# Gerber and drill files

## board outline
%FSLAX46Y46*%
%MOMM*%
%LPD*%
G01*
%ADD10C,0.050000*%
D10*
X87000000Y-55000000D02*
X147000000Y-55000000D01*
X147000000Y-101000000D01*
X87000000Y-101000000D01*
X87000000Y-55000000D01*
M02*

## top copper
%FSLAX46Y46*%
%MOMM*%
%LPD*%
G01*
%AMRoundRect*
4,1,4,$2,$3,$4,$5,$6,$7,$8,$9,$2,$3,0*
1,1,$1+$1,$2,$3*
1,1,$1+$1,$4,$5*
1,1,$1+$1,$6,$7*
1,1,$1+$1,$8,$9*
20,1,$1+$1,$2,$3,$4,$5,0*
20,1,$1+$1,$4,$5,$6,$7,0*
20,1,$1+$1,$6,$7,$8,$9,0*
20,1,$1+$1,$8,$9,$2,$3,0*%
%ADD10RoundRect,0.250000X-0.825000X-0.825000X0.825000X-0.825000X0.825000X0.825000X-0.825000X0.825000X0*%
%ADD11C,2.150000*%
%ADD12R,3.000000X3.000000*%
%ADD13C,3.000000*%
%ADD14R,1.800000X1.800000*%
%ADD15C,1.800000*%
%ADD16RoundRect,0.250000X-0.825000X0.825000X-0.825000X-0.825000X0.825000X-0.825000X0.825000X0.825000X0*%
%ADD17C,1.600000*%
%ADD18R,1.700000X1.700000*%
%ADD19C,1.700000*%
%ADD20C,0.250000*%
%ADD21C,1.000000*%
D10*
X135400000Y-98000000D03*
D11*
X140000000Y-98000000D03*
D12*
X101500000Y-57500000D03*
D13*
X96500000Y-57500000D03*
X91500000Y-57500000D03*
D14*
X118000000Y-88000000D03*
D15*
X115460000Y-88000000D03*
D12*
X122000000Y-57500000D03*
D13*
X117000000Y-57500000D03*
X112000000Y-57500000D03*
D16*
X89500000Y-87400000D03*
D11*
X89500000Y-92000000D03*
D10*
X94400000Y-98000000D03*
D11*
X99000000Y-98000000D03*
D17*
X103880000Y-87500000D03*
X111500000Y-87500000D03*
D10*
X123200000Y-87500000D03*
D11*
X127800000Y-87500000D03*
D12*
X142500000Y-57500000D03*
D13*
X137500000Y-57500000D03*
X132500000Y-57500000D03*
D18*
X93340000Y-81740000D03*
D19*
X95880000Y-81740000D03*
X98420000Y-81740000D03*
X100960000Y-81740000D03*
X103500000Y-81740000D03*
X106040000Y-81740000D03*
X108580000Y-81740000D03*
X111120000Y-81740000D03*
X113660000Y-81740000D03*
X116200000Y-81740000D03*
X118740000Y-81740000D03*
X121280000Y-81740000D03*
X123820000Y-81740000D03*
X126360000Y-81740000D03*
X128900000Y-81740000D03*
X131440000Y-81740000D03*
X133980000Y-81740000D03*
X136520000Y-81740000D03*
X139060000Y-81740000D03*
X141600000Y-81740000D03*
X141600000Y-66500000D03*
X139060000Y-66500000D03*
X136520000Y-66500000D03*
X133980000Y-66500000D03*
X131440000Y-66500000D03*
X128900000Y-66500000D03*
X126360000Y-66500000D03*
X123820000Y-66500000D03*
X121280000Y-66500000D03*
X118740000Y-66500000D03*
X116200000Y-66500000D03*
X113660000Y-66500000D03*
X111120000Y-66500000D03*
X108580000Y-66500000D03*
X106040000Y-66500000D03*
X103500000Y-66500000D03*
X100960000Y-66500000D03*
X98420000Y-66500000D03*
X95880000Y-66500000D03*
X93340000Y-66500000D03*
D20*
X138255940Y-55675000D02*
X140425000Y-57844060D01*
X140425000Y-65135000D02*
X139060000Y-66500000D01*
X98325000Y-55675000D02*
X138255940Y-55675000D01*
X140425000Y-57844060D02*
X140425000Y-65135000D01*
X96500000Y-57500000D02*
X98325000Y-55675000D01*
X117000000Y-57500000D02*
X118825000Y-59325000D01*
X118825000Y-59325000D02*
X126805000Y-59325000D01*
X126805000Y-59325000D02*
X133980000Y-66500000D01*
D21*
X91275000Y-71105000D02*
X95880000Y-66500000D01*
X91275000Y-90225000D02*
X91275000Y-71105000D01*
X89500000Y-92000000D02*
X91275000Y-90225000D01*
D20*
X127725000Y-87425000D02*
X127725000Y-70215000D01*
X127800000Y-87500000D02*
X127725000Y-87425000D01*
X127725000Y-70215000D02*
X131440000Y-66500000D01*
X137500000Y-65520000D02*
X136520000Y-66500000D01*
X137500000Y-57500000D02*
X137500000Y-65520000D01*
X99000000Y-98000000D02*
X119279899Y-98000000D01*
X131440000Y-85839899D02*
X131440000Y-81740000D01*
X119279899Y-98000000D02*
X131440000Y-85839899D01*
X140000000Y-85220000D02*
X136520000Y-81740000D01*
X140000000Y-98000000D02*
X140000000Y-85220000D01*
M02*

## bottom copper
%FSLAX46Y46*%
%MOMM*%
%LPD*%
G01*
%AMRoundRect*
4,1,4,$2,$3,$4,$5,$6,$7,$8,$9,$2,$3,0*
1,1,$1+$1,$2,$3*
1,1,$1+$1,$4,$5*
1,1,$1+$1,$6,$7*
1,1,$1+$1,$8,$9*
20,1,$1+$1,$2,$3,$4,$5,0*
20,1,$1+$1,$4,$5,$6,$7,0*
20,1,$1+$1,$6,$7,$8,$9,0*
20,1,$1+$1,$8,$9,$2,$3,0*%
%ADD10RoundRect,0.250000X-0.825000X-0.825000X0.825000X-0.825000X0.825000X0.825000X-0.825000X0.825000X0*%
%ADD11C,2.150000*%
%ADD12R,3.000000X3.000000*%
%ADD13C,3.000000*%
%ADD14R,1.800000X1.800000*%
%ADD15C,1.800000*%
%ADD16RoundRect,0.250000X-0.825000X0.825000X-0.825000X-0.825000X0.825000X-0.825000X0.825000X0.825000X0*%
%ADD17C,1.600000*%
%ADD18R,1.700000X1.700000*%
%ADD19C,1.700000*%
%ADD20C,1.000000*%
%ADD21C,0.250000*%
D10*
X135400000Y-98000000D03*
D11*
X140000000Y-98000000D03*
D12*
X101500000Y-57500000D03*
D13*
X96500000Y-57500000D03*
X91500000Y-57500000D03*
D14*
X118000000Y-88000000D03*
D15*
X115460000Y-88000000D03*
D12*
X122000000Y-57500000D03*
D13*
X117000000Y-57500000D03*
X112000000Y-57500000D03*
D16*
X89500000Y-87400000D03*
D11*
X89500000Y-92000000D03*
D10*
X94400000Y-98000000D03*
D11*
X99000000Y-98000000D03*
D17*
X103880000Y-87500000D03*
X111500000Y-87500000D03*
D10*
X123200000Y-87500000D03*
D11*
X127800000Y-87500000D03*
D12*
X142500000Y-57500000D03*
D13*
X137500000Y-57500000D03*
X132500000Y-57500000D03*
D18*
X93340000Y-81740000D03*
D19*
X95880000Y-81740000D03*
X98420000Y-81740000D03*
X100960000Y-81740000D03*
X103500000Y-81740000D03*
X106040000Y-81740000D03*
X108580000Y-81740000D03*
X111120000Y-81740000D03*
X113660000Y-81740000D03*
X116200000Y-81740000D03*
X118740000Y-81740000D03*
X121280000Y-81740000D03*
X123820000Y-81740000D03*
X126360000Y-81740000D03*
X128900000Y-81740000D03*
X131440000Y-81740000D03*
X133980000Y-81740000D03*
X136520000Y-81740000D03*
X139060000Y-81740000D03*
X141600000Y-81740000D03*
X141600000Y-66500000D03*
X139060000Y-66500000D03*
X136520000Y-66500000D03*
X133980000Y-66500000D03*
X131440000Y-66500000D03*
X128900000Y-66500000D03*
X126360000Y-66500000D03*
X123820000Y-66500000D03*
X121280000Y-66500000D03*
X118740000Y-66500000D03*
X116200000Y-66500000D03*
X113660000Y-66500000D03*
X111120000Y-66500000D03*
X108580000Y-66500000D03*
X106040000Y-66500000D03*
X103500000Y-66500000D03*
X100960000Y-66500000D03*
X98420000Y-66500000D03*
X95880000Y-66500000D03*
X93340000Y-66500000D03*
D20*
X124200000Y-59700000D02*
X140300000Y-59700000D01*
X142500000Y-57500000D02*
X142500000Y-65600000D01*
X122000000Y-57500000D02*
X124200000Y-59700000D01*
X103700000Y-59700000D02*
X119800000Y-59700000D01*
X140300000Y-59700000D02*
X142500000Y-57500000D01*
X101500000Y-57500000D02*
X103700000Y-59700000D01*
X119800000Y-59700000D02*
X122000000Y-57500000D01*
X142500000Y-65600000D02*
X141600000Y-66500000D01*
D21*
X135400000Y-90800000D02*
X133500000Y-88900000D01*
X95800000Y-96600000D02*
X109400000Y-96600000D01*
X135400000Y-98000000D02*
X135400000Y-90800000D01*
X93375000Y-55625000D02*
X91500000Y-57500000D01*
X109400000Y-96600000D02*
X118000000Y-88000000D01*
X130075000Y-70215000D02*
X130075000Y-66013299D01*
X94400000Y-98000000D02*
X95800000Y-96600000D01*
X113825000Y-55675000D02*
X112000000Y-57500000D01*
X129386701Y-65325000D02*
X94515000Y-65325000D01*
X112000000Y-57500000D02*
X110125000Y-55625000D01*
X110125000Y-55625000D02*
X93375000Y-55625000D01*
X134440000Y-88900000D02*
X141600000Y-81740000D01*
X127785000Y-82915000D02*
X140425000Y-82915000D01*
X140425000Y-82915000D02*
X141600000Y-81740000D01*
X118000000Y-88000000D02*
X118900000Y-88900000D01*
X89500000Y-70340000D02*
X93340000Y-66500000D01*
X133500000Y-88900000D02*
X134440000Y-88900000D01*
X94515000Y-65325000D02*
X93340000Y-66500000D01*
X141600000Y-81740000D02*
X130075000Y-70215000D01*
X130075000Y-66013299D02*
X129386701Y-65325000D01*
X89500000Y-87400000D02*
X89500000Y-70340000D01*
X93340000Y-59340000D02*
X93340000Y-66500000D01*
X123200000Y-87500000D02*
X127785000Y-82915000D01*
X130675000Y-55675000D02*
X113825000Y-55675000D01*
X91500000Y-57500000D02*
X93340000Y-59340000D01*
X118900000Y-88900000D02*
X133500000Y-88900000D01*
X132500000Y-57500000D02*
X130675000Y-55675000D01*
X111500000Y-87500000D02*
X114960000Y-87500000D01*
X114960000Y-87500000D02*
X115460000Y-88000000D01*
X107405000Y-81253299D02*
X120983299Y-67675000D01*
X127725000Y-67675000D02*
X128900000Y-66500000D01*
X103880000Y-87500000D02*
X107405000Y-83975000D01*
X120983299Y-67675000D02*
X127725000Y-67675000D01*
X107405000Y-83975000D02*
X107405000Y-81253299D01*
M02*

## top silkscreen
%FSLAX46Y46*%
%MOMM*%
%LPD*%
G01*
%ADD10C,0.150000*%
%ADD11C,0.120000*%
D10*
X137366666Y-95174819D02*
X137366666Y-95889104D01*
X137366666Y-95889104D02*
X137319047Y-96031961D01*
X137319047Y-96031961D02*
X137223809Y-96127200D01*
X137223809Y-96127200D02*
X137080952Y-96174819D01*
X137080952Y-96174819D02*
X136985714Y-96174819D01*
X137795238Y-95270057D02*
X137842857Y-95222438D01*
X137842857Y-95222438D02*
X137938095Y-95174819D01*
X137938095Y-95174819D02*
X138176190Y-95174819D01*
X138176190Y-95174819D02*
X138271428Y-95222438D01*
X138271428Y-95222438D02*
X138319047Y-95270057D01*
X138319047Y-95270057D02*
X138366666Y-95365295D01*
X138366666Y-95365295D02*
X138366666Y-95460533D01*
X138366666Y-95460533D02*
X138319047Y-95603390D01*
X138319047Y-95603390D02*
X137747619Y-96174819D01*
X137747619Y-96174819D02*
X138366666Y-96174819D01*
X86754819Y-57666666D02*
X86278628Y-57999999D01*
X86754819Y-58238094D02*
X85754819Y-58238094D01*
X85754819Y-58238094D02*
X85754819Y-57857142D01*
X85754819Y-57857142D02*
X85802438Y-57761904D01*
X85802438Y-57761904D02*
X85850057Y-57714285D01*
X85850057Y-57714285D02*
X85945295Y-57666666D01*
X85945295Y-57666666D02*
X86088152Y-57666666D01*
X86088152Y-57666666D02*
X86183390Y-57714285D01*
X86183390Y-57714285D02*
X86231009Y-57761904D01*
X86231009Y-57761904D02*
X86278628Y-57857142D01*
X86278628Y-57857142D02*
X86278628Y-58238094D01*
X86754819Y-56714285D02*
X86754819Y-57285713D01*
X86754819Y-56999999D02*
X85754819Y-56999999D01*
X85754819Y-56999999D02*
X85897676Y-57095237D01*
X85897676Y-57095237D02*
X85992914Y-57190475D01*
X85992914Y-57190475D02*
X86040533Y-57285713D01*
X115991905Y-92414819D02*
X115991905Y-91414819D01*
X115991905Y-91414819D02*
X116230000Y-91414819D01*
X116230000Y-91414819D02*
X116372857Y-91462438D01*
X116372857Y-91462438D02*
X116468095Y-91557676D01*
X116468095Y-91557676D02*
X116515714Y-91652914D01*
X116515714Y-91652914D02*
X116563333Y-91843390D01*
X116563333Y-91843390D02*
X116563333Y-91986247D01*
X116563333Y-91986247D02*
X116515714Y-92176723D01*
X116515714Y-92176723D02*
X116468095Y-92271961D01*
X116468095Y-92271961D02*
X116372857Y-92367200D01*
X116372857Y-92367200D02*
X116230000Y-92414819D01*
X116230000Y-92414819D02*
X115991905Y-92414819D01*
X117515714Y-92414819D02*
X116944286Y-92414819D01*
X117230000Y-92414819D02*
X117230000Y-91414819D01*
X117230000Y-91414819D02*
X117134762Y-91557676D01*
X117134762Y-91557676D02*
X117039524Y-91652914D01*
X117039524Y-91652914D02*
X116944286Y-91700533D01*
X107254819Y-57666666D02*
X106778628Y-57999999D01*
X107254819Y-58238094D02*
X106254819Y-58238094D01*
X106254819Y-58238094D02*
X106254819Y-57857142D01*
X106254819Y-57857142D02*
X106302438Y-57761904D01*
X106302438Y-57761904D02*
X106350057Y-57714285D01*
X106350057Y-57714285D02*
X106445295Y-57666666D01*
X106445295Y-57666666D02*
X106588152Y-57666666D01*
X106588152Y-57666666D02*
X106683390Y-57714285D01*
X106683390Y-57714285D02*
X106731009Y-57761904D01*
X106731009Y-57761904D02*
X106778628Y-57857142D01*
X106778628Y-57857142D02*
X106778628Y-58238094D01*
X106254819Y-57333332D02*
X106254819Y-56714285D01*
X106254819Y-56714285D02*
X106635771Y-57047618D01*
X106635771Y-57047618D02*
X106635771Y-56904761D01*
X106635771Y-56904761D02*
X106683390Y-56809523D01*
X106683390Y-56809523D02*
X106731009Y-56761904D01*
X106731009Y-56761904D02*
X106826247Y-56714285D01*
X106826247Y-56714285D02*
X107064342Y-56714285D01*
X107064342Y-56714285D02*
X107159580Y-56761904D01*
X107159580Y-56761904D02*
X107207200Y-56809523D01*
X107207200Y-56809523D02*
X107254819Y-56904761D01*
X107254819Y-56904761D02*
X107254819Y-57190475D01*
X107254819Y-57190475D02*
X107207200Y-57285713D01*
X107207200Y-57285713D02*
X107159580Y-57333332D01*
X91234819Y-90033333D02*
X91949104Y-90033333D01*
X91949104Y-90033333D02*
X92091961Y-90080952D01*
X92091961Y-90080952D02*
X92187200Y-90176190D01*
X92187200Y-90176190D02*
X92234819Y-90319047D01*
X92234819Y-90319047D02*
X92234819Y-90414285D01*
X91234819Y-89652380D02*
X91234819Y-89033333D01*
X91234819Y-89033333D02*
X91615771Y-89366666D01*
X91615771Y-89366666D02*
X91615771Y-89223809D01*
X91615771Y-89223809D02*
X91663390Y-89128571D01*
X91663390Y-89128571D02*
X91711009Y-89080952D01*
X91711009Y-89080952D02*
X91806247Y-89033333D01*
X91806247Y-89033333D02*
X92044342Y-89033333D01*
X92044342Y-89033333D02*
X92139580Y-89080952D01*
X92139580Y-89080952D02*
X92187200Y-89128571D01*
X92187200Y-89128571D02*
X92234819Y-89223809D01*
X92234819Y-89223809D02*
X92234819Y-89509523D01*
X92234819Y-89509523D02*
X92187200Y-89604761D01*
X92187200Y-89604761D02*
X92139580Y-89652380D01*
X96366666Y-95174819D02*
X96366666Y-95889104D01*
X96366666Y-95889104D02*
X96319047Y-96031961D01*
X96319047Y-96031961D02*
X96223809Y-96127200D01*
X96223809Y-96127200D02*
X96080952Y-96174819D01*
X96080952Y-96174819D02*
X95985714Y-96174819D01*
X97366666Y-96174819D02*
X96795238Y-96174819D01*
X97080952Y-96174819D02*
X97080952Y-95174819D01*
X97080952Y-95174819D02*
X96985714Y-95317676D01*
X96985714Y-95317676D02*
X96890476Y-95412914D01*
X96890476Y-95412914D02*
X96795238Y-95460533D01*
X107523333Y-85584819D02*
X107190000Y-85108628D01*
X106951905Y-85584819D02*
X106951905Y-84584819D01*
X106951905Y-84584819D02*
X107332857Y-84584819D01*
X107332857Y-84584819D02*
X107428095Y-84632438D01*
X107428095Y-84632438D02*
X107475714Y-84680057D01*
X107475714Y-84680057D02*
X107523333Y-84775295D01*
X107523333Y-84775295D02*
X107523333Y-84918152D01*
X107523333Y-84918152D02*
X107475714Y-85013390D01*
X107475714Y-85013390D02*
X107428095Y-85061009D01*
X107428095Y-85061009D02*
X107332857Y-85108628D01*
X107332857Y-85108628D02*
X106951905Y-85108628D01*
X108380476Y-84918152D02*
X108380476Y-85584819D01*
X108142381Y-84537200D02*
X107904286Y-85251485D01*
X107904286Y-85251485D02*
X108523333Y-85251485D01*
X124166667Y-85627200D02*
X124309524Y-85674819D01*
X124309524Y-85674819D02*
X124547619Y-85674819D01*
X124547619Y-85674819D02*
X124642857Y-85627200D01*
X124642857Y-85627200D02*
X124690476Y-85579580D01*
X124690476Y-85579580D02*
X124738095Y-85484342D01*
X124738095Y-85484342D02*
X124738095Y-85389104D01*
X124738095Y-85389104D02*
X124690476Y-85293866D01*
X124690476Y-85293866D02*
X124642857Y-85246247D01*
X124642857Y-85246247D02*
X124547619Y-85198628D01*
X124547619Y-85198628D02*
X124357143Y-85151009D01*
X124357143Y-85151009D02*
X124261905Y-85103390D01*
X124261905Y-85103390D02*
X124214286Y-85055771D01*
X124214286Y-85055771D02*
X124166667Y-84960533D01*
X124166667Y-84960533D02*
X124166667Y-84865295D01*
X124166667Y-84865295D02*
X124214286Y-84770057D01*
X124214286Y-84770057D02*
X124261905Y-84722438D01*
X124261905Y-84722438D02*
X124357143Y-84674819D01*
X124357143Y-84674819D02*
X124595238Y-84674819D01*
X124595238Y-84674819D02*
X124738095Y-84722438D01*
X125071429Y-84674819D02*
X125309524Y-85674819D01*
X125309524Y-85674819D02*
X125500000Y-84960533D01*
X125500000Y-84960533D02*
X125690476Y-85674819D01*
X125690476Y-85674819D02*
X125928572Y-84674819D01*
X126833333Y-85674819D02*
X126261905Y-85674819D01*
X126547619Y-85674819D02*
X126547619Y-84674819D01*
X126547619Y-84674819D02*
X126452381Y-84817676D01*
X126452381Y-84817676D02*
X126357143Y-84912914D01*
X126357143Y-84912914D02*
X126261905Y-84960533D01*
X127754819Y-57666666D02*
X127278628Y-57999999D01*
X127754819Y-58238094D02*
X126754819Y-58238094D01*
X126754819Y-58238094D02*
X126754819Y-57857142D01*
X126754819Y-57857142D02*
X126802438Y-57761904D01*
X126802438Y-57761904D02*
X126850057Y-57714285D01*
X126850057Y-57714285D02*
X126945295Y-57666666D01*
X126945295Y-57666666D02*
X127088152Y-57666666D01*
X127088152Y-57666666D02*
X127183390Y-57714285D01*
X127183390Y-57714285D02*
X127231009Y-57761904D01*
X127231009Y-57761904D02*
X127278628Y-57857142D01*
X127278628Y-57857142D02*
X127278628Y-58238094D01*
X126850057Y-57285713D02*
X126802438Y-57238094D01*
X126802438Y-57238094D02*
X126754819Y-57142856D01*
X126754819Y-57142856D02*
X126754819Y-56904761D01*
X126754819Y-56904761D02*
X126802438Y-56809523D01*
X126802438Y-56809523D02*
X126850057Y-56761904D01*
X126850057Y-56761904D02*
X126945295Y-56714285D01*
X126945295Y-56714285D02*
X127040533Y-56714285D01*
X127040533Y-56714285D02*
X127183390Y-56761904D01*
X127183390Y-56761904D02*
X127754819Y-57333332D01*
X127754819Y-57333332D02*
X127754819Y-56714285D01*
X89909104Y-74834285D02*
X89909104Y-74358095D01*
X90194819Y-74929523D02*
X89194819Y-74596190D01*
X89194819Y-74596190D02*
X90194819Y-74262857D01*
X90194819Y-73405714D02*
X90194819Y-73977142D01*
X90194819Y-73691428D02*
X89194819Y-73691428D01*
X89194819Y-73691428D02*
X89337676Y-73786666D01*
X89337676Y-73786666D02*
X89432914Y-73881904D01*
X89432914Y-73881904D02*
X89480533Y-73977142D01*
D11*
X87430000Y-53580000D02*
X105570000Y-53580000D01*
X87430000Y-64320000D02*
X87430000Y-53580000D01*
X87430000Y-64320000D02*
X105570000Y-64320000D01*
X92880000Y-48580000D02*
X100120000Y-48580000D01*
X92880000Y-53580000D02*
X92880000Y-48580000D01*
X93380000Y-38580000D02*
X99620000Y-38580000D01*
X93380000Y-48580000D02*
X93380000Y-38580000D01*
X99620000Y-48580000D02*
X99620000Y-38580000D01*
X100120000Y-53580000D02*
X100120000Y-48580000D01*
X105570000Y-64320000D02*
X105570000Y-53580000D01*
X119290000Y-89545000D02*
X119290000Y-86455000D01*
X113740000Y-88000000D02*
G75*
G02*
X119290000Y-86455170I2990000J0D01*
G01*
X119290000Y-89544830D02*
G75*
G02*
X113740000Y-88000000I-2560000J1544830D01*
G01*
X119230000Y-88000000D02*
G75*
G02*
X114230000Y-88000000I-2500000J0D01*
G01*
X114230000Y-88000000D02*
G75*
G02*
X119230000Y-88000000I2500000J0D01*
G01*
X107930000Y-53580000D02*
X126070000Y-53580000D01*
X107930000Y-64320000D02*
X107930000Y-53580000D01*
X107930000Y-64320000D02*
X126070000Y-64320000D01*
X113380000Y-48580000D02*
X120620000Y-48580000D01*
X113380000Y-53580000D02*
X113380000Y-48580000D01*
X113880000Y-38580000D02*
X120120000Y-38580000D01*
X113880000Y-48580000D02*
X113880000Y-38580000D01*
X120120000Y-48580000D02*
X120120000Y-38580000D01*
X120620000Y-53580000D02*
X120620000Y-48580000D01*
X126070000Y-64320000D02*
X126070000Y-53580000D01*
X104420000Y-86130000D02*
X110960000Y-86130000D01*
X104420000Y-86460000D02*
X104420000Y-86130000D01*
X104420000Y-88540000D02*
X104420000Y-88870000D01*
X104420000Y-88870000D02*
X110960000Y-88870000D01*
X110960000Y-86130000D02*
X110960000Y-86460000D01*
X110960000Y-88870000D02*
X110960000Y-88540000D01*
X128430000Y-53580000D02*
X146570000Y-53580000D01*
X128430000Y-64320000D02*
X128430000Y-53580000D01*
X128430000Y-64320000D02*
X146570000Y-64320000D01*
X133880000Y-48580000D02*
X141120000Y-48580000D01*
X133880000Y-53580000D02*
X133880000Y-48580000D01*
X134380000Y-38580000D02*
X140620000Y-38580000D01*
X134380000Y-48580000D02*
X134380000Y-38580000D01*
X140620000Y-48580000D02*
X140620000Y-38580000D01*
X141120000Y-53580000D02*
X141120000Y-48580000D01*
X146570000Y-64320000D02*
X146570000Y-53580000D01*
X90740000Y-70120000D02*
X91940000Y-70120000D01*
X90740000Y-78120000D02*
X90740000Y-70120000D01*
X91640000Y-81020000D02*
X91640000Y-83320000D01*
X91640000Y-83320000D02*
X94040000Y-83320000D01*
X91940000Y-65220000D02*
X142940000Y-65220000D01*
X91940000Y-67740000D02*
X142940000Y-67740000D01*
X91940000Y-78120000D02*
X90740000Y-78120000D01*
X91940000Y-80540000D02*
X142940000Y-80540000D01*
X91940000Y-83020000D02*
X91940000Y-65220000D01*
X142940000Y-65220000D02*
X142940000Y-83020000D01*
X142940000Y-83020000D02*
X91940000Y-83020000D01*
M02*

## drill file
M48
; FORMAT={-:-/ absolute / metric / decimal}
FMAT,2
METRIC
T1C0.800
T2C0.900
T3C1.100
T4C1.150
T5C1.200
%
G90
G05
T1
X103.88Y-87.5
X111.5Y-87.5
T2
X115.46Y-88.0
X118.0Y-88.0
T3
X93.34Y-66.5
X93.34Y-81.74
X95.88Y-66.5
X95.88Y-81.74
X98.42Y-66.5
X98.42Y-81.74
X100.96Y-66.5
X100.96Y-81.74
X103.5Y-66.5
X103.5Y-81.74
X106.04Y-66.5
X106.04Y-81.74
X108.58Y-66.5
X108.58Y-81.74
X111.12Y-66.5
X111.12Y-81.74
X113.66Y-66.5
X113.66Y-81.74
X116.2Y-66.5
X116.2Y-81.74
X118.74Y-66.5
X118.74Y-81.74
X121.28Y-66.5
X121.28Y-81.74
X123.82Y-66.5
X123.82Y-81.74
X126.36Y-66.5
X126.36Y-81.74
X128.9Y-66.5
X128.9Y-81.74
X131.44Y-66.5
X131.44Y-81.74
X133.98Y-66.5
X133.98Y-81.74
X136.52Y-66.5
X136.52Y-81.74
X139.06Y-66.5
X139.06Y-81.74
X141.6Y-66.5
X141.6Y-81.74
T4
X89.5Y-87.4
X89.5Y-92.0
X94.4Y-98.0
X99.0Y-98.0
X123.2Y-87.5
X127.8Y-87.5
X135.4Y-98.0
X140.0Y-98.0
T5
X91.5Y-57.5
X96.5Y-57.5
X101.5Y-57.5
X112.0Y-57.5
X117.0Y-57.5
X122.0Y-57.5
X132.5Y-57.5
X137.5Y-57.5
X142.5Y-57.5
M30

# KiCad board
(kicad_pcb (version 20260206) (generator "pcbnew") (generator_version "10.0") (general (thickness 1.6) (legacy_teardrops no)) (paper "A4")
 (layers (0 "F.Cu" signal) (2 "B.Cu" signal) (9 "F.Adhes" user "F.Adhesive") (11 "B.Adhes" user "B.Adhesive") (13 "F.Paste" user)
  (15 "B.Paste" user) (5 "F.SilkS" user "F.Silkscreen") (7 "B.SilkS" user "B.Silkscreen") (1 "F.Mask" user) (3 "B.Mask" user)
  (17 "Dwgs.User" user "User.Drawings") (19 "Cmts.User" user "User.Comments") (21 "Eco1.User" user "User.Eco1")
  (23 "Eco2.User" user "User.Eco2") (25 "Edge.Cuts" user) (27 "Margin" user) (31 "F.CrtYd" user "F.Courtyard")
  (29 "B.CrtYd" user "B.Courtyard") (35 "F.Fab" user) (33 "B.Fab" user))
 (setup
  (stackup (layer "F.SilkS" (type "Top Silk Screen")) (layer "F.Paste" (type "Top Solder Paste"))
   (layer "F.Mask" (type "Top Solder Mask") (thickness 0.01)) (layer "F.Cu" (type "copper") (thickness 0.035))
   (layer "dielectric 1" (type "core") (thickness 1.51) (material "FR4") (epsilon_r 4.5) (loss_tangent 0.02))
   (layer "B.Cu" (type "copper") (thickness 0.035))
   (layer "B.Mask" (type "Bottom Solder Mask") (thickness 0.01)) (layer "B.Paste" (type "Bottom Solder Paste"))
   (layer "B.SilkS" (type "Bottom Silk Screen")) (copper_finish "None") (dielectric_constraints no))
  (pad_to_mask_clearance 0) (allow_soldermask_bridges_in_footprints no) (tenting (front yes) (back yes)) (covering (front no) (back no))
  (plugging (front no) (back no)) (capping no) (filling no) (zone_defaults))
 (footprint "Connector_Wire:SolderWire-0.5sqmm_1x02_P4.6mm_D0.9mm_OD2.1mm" (layer "F.Cu") (at 135.4 98)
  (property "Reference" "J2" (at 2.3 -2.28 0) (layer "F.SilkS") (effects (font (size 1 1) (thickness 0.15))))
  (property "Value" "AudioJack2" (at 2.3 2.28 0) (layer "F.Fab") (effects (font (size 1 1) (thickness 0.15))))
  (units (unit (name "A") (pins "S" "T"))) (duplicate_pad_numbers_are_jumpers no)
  (pad "S" thru_hole roundrect (at 0 0) (size 2.15 2.15) (drill 1.15) (layers "*.Cu" "*.Mask") (remove_unused_layers no)
   (roundrect_rratio 0.116279) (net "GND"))
  (pad "T" thru_hole circle (at 4.6 0) (size 2.15 2.15) (drill 1.15) (layers "*.Cu" "*.Mask") (remove_unused_layers no)
   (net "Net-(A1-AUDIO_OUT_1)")))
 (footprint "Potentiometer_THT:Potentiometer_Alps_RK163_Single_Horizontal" (layer "F.Cu") (at 101.5 57.5 -90)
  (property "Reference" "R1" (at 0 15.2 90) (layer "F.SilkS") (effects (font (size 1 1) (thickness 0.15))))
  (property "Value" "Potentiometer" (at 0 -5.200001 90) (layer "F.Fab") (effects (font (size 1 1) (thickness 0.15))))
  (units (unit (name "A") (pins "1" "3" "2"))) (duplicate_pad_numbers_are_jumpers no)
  (fp_line (start -3.92 14.07) (end -3.92 -4.07) (stroke (width 0.12) (type solid)) (layer "F.SilkS"))
  (fp_line (start 6.82 14.07) (end -3.92 14.07) (stroke (width 0.12) (type solid)) (layer "F.SilkS"))
  (fp_line (start 6.82 14.07) (end 6.82 -4.07) (stroke (width 0.12) (type solid)) (layer "F.SilkS"))
  (fp_line (start -8.92 8.62) (end -8.92 1.38) (stroke (width 0.12) (type solid)) (layer "F.SilkS"))
  (fp_line (start -3.92 8.62) (end -8.92 8.62) (stroke (width 0.12) (type solid)) (layer "F.SilkS"))
  (fp_line (start -18.92 8.12) (end -18.92 1.88) (stroke (width 0.12) (type solid)) (layer "F.SilkS"))
  (fp_line (start -8.92 8.12) (end -18.92 8.12) (stroke (width 0.12) (type solid)) (layer "F.SilkS"))
  (fp_line (start -8.92 1.88) (end -18.92 1.88) (stroke (width 0.12) (type solid)) (layer "F.SilkS"))
  (fp_line (start -3.92 1.38) (end -8.92 1.38) (stroke (width 0.12) (type solid)) (layer "F.SilkS"))
  (fp_line (start 6.82 -4.07) (end -3.92 -4.07) (stroke (width 0.12) (type solid)) (layer "F.SilkS"))
  (pad "1" thru_hole rect (at 0 0 90) (size 3 3) (drill 1.2) (layers "*.Cu" "*.Mask") (remove_unused_layers no) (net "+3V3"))
  (pad "2" thru_hole circle (at 0 5 90) (size 3 3) (drill 1.2) (layers "*.Cu" "*.Mask") (remove_unused_layers no) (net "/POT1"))
  (pad "3" thru_hole circle (at 0 10 90) (size 3 3) (drill 1.2) (layers "*.Cu" "*.Mask") (remove_unused_layers no) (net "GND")))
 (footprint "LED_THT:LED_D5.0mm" (layer "F.Cu") (at 118 88 180)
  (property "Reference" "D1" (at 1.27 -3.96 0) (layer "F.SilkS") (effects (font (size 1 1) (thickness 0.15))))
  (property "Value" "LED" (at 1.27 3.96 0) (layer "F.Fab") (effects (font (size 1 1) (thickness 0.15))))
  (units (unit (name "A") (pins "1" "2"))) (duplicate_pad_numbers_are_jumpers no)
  (fp_line (start -1.29 -1.545) (end -1.29 1.545) (stroke (width 0.12) (type solid)) (layer "F.SilkS"))
  (fp_arc (start 4.26 0) (mid 2.071779 2.880495) (end -1.29 1.54483) (stroke (width 0.12) (type solid)) (layer "F.SilkS"))
  (fp_arc (start -1.29 -1.54483) (mid 2.071779 -2.880495) (end 4.26 0) (stroke (width 0.12) (type solid)) (layer "F.SilkS"))
  (fp_circle (center 1.27 0) (end 3.77 0) (stroke (width 0.12) (type solid)) (fill no) (layer "F.SilkS"))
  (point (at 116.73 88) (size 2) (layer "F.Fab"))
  (pad "1" thru_hole rect (at 0 0 180) (size 1.8 1.8) (drill 0.9) (layers "*.Cu" "*.Mask") (remove_unused_layers no) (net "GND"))
  (pad "2" thru_hole circle (at 2.54 0 180) (size 1.8 1.8) (drill 0.9) (layers "*.Cu" "*.Mask") (remove_unused_layers no) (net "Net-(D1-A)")))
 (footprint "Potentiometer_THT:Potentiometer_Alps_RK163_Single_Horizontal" (layer "F.Cu") (at 122 57.5 -90)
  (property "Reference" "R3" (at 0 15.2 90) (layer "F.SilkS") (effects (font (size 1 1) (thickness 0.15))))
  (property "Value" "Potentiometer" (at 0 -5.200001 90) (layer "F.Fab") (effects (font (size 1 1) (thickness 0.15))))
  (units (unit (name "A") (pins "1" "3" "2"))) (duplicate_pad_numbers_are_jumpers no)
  (fp_line (start -3.92 14.07) (end -3.92 -4.07) (stroke (width 0.12) (type solid)) (layer "F.SilkS"))
  (fp_line (start 6.82 14.07) (end -3.92 14.07) (stroke (width 0.12) (type solid)) (layer "F.SilkS"))
  (fp_line (start 6.82 14.07) (end 6.82 -4.07) (stroke (width 0.12) (type solid)) (layer "F.SilkS"))
  (fp_line (start -8.92 8.62) (end -8.92 1.38) (stroke (width 0.12) (type solid)) (layer "F.SilkS"))
  (fp_line (start -3.92 8.62) (end -8.92 8.62) (stroke (width 0.12) (type solid)) (layer "F.SilkS"))
  (fp_line (start -18.92 8.12) (end -18.92 1.88) (stroke (width 0.12) (type solid)) (layer "F.SilkS"))
  (fp_line (start -8.92 8.12) (end -18.92 8.12) (stroke (width 0.12) (type solid)) (layer "F.SilkS"))
  (fp_line (start -8.92 1.88) (end -18.92 1.88) (stroke (width 0.12) (type solid)) (layer "F.SilkS"))
  (fp_line (start -3.92 1.38) (end -8.92 1.38) (stroke (width 0.12) (type solid)) (layer "F.SilkS"))
  (fp_line (start 6.82 -4.07) (end -3.92 -4.07) (stroke (width 0.12) (type solid)) (layer "F.SilkS"))
  (pad "1" thru_hole rect (at 0 0 90) (size 3 3) (drill 1.2) (layers "*.Cu" "*.Mask") (remove_unused_layers no) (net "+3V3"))
  (pad "2" thru_hole circle (at 0 5 90) (size 3 3) (drill 1.2) (layers "*.Cu" "*.Mask") (remove_unused_layers no) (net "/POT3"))
  (pad "3" thru_hole circle (at 0 10 90) (size 3 3) (drill 1.2) (layers "*.Cu" "*.Mask") (remove_unused_layers no) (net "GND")))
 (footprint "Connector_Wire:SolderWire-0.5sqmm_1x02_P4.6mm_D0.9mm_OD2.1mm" (layer "F.Cu") (at 89.5 87.4 -90)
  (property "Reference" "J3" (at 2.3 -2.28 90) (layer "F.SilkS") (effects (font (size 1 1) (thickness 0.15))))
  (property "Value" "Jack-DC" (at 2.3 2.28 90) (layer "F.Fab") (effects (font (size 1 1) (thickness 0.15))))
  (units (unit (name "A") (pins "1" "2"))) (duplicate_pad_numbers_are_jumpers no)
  (pad "1" thru_hole roundrect (at 0 0 270) (size 2.15 2.15) (drill 1.15) (layers "*.Cu" "*.Mask") (remove_unused_layers no)
   (roundrect_rratio 0.116279) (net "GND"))
  (pad "2" thru_hole circle (at 4.6 0 270) (size 2.15 2.15) (drill 1.15) (layers "*.Cu" "*.Mask") (remove_unused_layers no)
   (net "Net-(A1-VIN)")))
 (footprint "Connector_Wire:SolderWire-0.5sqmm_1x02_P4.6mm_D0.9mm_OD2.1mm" (layer "F.Cu") (at 94.4 98)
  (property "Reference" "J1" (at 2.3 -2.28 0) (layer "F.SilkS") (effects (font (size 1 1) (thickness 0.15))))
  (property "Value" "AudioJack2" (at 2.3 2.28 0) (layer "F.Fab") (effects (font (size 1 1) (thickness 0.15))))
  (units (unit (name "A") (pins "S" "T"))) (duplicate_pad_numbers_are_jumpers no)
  (pad "S" thru_hole roundrect (at 0 0) (size 2.15 2.15) (drill 1.15) (layers "*.Cu" "*.Mask") (remove_unused_layers no)
   (roundrect_rratio 0.116279) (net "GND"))
  (pad "T" thru_hole circle (at 4.6 0) (size 2.15 2.15) (drill 1.15) (layers "*.Cu" "*.Mask") (remove_unused_layers no)
   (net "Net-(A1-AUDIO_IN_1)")))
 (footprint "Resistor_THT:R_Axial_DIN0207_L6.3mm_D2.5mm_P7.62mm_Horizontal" (layer "F.Cu") (at 103.88 87.5)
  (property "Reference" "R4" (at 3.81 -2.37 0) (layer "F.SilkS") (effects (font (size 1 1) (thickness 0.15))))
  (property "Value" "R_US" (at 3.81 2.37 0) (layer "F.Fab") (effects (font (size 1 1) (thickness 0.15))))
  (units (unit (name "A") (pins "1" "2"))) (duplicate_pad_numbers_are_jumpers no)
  (fp_line (start 0.54 -1.37) (end 7.08 -1.37) (stroke (width 0.12) (type solid)) (layer "F.SilkS"))
  (fp_line (start 0.54 -1.04) (end 0.54 -1.37) (stroke (width 0.12) (type solid)) (layer "F.SilkS"))
  (fp_line (start 0.54 1.04) (end 0.54 1.37) (stroke (width 0.12) (type solid)) (layer "F.SilkS"))
  (fp_line (start 0.54 1.37) (end 7.08 1.37) (stroke (width 0.12) (type solid)) (layer "F.SilkS"))
  (fp_line (start 7.08 -1.37) (end 7.08 -1.04) (stroke (width 0.12) (type solid)) (layer "F.SilkS"))
  (fp_line (start 7.08 1.37) (end 7.08 1.04) (stroke (width 0.12) (type solid)) (layer "F.SilkS"))
  (pad "1" thru_hole circle (at 0 0) (size 1.6 1.6) (drill 0.8) (layers "*.Cu" "*.Mask") (remove_unused_layers no) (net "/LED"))
  (pad "2" thru_hole circle (at 7.62 0) (size 1.6 1.6) (drill 0.8) (layers "*.Cu" "*.Mask") (remove_unused_layers no) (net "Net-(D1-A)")))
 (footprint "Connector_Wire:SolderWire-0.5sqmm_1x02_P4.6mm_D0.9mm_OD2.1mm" (layer "F.Cu") (at 123.2 87.5)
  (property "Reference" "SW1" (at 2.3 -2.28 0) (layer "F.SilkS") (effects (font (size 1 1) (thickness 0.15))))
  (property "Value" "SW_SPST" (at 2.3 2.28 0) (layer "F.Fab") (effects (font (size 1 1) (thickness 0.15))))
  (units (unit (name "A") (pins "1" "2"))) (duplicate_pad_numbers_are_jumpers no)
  (pad "1" thru_hole roundrect (at 0 0) (size 2.15 2.15) (drill 1.15) (layers "*.Cu" "*.Mask") (remove_unused_layers no)
   (roundrect_rratio 0.116279) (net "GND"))
  (pad "2" thru_hole circle (at 4.6 0) (size 2.15 2.15) (drill 1.15) (layers "*.Cu" "*.Mask") (remove_unused_layers no) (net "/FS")))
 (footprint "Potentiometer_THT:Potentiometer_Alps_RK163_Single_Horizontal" (layer "F.Cu") (at 142.5 57.5 -90)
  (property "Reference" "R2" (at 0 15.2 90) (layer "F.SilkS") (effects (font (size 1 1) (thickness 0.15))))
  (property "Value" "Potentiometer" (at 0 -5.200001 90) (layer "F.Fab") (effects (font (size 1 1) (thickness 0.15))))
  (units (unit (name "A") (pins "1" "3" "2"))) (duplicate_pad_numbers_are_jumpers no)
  (fp_line (start -3.92 14.07) (end -3.92 -4.07) (stroke (width 0.12) (type solid)) (layer "F.SilkS"))
  (fp_line (start 6.82 14.07) (end -3.92 14.07) (stroke (width 0.12) (type solid)) (layer "F.SilkS"))
  (fp_line (start 6.82 14.07) (end 6.82 -4.07) (stroke (width 0.12) (type solid)) (layer "F.SilkS"))
  (fp_line (start -8.92 8.62) (end -8.92 1.38) (stroke (width 0.12) (type solid)) (layer "F.SilkS"))
  (fp_line (start -3.92 8.62) (end -8.92 8.62) (stroke (width 0.12) (type solid)) (layer "F.SilkS"))
  (fp_line (start -18.92 8.12) (end -18.92 1.88) (stroke (width 0.12) (type solid)) (layer "F.SilkS"))
  (fp_line (start -8.92 8.12) (end -18.92 8.12) (stroke (width 0.12) (type solid)) (layer "F.SilkS"))
  (fp_line (start -8.92 1.88) (end -18.92 1.88) (stroke (width 0.12) (type solid)) (layer "F.SilkS"))
  (fp_line (start -3.92 1.38) (end -8.92 1.38) (stroke (width 0.12) (type solid)) (layer "F.SilkS"))
  (fp_line (start 6.82 -4.07) (end -3.92 -4.07) (stroke (width 0.12) (type solid)) (layer "F.SilkS"))
  (pad "1" thru_hole rect (at 0 0 90) (size 3 3) (drill 1.2) (layers "*.Cu" "*.Mask") (remove_unused_layers no) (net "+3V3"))
  (pad "2" thru_hole circle (at 0 5 90) (size 3 3) (drill 1.2) (layers "*.Cu" "*.Mask") (remove_unused_layers no) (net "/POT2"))
  (pad "3" thru_hole circle (at 0 10 90) (size 3 3) (drill 1.2) (layers "*.Cu" "*.Mask") (remove_unused_layers no) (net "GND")))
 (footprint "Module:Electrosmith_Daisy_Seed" (layer "F.Cu") (at 93.34 81.74 90)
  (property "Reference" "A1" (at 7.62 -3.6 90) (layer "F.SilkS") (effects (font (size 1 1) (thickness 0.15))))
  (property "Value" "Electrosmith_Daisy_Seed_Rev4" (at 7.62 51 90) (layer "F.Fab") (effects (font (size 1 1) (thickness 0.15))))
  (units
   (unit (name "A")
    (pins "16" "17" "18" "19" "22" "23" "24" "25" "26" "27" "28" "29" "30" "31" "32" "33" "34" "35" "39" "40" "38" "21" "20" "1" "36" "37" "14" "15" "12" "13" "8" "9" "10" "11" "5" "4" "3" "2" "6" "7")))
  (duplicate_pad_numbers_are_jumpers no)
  (fp_line (start 11.62 -2.6) (end 11.62 -1.4) (stroke (width 0.12) (type solid)) (layer "F.SilkS"))
  (fp_line (start 3.62 -2.6) (end 11.62 -2.6) (stroke (width 0.12) (type solid)) (layer "F.SilkS"))
  (fp_line (start 0.72 -1.7) (end -1.58 -1.7) (stroke (width 0.12) (type solid)) (layer "F.SilkS"))
  (fp_line (start -1.58 -1.7) (end -1.58 0.7) (stroke (width 0.12) (type solid)) (layer "F.SilkS"))
  (fp_line (start 16.52 -1.4) (end 16.52 49.6) (stroke (width 0.12) (type solid)) (layer "F.SilkS"))
  (fp_line (start 14 -1.4) (end 14 49.6) (stroke (width 0.12) (type solid)) (layer "F.SilkS"))
  (fp_line (start 3.62 -1.4) (end 3.62 -2.6) (stroke (width 0.12) (type solid)) (layer "F.SilkS"))
  (fp_line (start 1.2 -1.4) (end 1.2 49.6) (stroke (width 0.12) (type solid)) (layer "F.SilkS"))
  (fp_line (start -1.28 -1.4) (end 16.52 -1.4) (stroke (width 0.12) (type solid)) (layer "F.SilkS"))
  (fp_line (start 16.52 49.6) (end -1.28 49.6) (stroke (width 0.12) (type solid)) (layer "F.SilkS"))
  (fp_line (start -1.28 49.6) (end -1.28 -1.4) (stroke (width 0.12) (type solid)) (layer "F.SilkS"))
  (pad "1" thru_hole rect (at 0 0 90) (size 1.7 1.7) (drill 1.1) (layers "*.Cu" "*.Mask") (remove_unused_layers no)
   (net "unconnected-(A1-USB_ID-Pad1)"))
  (pad "2" thru_hole circle (at 0 2.54 90) (size 1.7 1.7) (drill 1.1) (layers "*.Cu" "*.Mask") (remove_unused_layers no)
   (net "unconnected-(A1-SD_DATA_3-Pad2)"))
  (pad "3" thru_hole circle (at 0 5.08 90) (size 1.7 1.7) (drill 1.1) (layers "*.Cu" "*.Mask") (remove_unused_layers no)
   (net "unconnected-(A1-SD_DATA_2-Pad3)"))
  (pad "4" thru_hole circle (at 0 7.62 90) (size 1.7 1.7) (drill 1.1) (layers "*.Cu" "*.Mask") (remove_unused_layers no)
   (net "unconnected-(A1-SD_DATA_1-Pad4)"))
  (pad "5" thru_hole circle (at 0 10.16 90) (size 1.7 1.7) (drill 1.1) (layers "*.Cu" "*.Mask") (remove_unused_layers no)
   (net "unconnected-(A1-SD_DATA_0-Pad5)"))
  (pad "6" thru_hole circle (at 0 12.7 90) (size 1.7 1.7) (drill 1.1) (layers "*.Cu" "*.Mask") (remove_unused_layers no)
   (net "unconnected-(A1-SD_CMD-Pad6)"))
  (pad "7" thru_hole circle (at 0 15.24 90) (size 1.7 1.7) (drill 1.1) (layers "*.Cu" "*.Mask") (remove_unused_layers no)
   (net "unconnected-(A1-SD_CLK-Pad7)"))
  (pad "8" thru_hole circle (at 0 17.78 90) (size 1.7 1.7) (drill 1.1) (layers "*.Cu" "*.Mask") (remove_unused_layers no)
   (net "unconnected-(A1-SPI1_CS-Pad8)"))
  (pad "9" thru_hole circle (at 0 20.32 90) (size 1.7 1.7) (drill 1.1) (layers "*.Cu" "*.Mask") (remove_unused_layers no)
   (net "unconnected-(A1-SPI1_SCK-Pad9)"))
  (pad "10" thru_hole circle (at 0 22.86 90) (size 1.7 1.7) (drill 1.1) (layers "*.Cu" "*.Mask") (remove_unused_layers no)
   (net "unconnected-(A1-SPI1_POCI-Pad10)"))
  (pad "11" thru_hole circle (at 0 25.4 90) (size 1.7 1.7) (drill 1.1) (layers "*.Cu" "*.Mask") (remove_unused_layers no)
   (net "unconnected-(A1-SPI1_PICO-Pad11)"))
  (pad "12" thru_hole circle (at 0 27.94 90) (size 1.7 1.7) (drill 1.1) (layers "*.Cu" "*.Mask") (remove_unused_layers no)
   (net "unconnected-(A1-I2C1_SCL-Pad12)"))
  (pad "13" thru_hole circle (at 0 30.48 90) (size 1.7 1.7) (drill 1.1) (layers "*.Cu" "*.Mask") (remove_unused_layers no)
   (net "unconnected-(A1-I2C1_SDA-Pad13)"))
  (pad "14" thru_hole circle (at 0 33.02 90) (size 1.7 1.7) (drill 1.1) (layers "*.Cu" "*.Mask") (remove_unused_layers no)
   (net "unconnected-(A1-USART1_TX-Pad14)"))
  (pad "15" thru_hole circle (at 0 35.56 90) (size 1.7 1.7) (drill 1.1) (layers "*.Cu" "*.Mask") (remove_unused_layers no)
   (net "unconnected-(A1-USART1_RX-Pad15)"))
  (pad "16" thru_hole circle (at 0 38.1 90) (size 1.7 1.7) (drill 1.1) (layers "*.Cu" "*.Mask") (remove_unused_layers no)
   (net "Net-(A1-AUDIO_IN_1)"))
  (pad "17" thru_hole circle (at 0 40.64 90) (size 1.7 1.7) (drill 1.1) (layers "*.Cu" "*.Mask") (remove_unused_layers no)
   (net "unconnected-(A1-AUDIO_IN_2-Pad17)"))
  (pad "18" thru_hole circle (at 0 43.18 90) (size 1.7 1.7) (drill 1.1) (layers "*.Cu" "*.Mask") (remove_unused_layers no)
   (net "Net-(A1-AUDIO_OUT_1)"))
  (pad "19" thru_hole circle (at 0 45.72 90) (size 1.7 1.7) (drill 1.1) (layers "*.Cu" "*.Mask") (remove_unused_layers no)
   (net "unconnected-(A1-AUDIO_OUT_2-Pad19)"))
  (pad "20" thru_hole circle (at 0 48.26 90) (size 1.7 1.7) (drill 1.1) (layers "*.Cu" "*.Mask") (remove_unused_layers no) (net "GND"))
  (pad "21" thru_hole circle (at 15.24 48.26 90) (size 1.7 1.7) (drill 1.1) (layers "*.Cu" "*.Mask") (remove_unused_layers no) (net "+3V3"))
  (pad "22" thru_hole circle (at 15.24 45.72 90) (size 1.7 1.7) (drill 1.1) (layers "*.Cu" "*.Mask") (remove_unused_layers no) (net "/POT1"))
  (pad "23" thru_hole circle (at 15.24 43.18 90) (size 1.7 1.7) (drill 1.1) (layers "*.Cu" "*.Mask") (remove_unused_layers no) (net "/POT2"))
  (pad "24" thru_hole circle (at 15.24 40.64 90) (size 1.7 1.7) (drill 1.1) (layers "*.Cu" "*.Mask") (remove_unused_layers no) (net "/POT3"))
  (pad "25" thru_hole circle (at 15.24 38.1 90) (size 1.7 1.7) (drill 1.1) (layers "*.Cu" "*.Mask") (remove_unused_layers no) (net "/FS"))
  (pad "26" thru_hole circle (at 15.24 35.56 90) (size 1.7 1.7) (drill 1.1) (layers "*.Cu" "*.Mask") (remove_unused_layers no) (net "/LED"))
  (pad "27" thru_hole circle (at 15.24 33.02 90) (size 1.7 1.7) (drill 1.1) (layers "*.Cu" "*.Mask") (remove_unused_layers no)
   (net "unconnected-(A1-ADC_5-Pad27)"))
  (pad "28" thru_hole circle (at 15.24 30.48 90) (size 1.7 1.7) (drill 1.1) (layers "*.Cu" "*.Mask") (remove_unused_layers no)
   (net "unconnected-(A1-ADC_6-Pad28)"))
  (pad "29" thru_hole circle (at 15.24 27.94 90) (size 1.7 1.7) (drill 1.1) (layers "*.Cu" "*.Mask") (remove_unused_layers no)
   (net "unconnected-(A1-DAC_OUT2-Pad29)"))
  (pad "30" thru_hole circle (at 15.24 25.4 90) (size 1.7 1.7) (drill 1.1) (layers "*.Cu" "*.Mask") (remove_unused_layers no)
   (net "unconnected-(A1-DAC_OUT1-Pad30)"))
  (pad "31" thru_hole circle (at 15.24 22.86 90) (size 1.7 1.7) (drill 1.1) (layers "*.Cu" "*.Mask") (remove_unused_layers no)
   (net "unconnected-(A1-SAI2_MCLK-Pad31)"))
  (pad "32" thru_hole circle (at 15.24 20.32 90) (size 1.7 1.7) (drill 1.1) (layers "*.Cu" "*.Mask") (remove_unused_layers no)
   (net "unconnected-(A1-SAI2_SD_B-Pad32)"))
  (pad "33" thru_hole circle (at 15.24 17.78 90) (size 1.7 1.7) (drill 1.1) (layers "*.Cu" "*.Mask") (remove_unused_layers no)
   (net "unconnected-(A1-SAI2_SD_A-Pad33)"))
  (pad "34" thru_hole circle (at 15.24 15.24 90) (size 1.7 1.7) (drill 1.1) (layers "*.Cu" "*.Mask") (remove_unused_layers no)
   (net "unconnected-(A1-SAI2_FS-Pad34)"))
  (pad "35" thru_hole circle (at 15.24 12.7 90) (size 1.7 1.7) (drill 1.1) (layers "*.Cu" "*.Mask") (remove_unused_layers no)
   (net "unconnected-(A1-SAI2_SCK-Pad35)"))
  (pad "36" thru_hole circle (at 15.24 10.16 90) (size 1.7 1.7) (drill 1.1) (layers "*.Cu" "*.Mask") (remove_unused_layers no)
   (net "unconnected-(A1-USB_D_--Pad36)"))
  (pad "37" thru_hole circle (at 15.24 7.62 90) (size 1.7 1.7) (drill 1.1) (layers "*.Cu" "*.Mask") (remove_unused_layers no)
   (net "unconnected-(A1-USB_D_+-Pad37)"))
  (pad "38" thru_hole circle (at 15.24 5.08 90) (size 1.7 1.7) (drill 1.1) (layers "*.Cu" "*.Mask") (remove_unused_layers no)
   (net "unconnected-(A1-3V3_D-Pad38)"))
  (pad "39" thru_hole circle (at 15.24 2.54 90) (size 1.7 1.7) (drill 1.1) (layers "*.Cu" "*.Mask") (remove_unused_layers no)
   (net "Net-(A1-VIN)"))
  (pad "40" thru_hole circle (at 15.24 0 90) (size 1.7 1.7) (drill 1.1) (layers "*.Cu" "*.Mask") (remove_unused_layers no) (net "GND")))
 (gr_rect (start 87 55) (end 147 101) (stroke (width 0.05) (type default)) (fill no) (layer "Edge.Cuts"))
 (segment (start 124.2 59.7) (end 140.3 59.7) (width 1) (layer "B.Cu") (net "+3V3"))
 (segment (start 142.5 57.5) (end 142.5 65.6) (width 1) (layer "B.Cu") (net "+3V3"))
 (segment (start 122 57.5) (end 124.2 59.7) (width 1) (layer "B.Cu") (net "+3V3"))
 (segment (start 103.7 59.7) (end 119.8 59.7) (width 1) (layer "B.Cu") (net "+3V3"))
 (segment (start 140.3 59.7) (end 142.5 57.5) (width 1) (layer "B.Cu") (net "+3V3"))
 (segment (start 101.5 57.5) (end 103.7 59.7) (width 1) (layer "B.Cu") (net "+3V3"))
 (segment (start 119.8 59.7) (end 122 57.5) (width 1) (layer "B.Cu") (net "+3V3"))
 (segment (start 142.5 65.6) (end 141.6 66.5) (width 1) (layer "B.Cu") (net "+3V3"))
 (segment (start 138.25594 55.675) (end 140.425 57.84406) (width 0.25) (layer "F.Cu") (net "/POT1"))
 (segment (start 140.425 65.135) (end 139.06 66.5) (width 0.25) (layer "F.Cu") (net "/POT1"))
 (segment (start 98.325 55.675) (end 138.25594 55.675) (width 0.25) (layer "F.Cu") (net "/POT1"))
 (segment (start 140.425 57.84406) (end 140.425 65.135) (width 0.25) (layer "F.Cu") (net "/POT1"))
 (segment (start 96.5 57.5) (end 98.325 55.675) (width 0.25) (layer "F.Cu") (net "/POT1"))
 (segment (start 135.4 90.8) (end 133.5 88.9) (width 0.25) (layer "B.Cu") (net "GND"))
 (segment (start 95.8 96.6) (end 109.4 96.6) (width 0.25) (layer "B.Cu") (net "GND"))
 (segment (start 135.4 98) (end 135.4 90.8) (width 0.25) (layer "B.Cu") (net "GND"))
 (segment (start 93.375 55.625) (end 91.5 57.5) (width 0.25) (layer "B.Cu") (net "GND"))
 (segment (start 109.4 96.6) (end 118 88) (width 0.25) (layer "B.Cu") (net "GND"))
 (segment (start 130.075 70.215) (end 130.075 66.013299) (width 0.25) (layer "B.Cu") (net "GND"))
 (segment (start 94.4 98) (end 95.8 96.6) (width 0.25) (layer "B.Cu") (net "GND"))
 (segment (start 113.825 55.675) (end 112 57.5) (width 0.25) (layer "B.Cu") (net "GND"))
 (segment (start 129.386701 65.325) (end 94.515 65.325) (width 0.25) (layer "B.Cu") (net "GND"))
 (segment (start 112 57.5) (end 110.125 55.625) (width 0.25) (layer "B.Cu") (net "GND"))
 (segment (start 110.125 55.625) (end 93.375 55.625) (width 0.25) (layer "B.Cu") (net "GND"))
 (segment (start 134.44 88.9) (end 141.6 81.74) (width 0.25) (layer "B.Cu") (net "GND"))
 (segment (start 127.785 82.915) (end 140.425 82.915) (width 0.25) (layer "B.Cu") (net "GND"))
 (segment (start 140.425 82.915) (end 141.6 81.74) (width 0.25) (layer "B.Cu") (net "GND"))
 (segment (start 118 88) (end 118.9 88.9) (width 0.25) (layer "B.Cu") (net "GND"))
 (segment (start 89.5 70.34) (end 93.34 66.5) (width 0.25) (layer "B.Cu") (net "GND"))
 (segment (start 133.5 88.9) (end 134.44 88.9) (width 0.25) (layer "B.Cu") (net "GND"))
 (segment (start 94.515 65.325) (end 93.34 66.5) (width 0.25) (layer "B.Cu") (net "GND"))
 (segment (start 141.6 81.74) (end 130.075 70.215) (width 0.25) (layer "B.Cu") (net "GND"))
 (segment (start 130.075 66.013299) (end 129.386701 65.325) (width 0.25) (layer "B.Cu") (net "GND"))
 (segment (start 89.5 87.4) (end 89.5 70.34) (width 0.25) (layer "B.Cu") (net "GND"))
 (segment (start 93.34 59.34) (end 93.34 66.5) (width 0.25) (layer "B.Cu") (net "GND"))
 (segment (start 123.2 87.5) (end 127.785 82.915) (width 0.25) (layer "B.Cu") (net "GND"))
 (segment (start 130.675 55.675) (end 113.825 55.675) (width 0.25) (layer "B.Cu") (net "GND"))
 (segment (start 91.5 57.5) (end 93.34 59.34) (width 0.25) (layer "B.Cu") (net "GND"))
 (segment (start 118.9 88.9) (end 133.5 88.9) (width 0.25) (layer "B.Cu") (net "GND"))
 (segment (start 132.5 57.5) (end 130.675 55.675) (width 0.25) (layer "B.Cu") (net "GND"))
 (segment (start 111.5 87.5) (end 114.96 87.5) (width 0.25) (layer "B.Cu") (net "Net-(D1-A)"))
 (segment (start 114.96 87.5) (end 115.46 88) (width 0.25) (layer "B.Cu") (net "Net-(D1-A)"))
 (segment (start 117 57.5) (end 118.825 59.325) (width 0.25) (layer "F.Cu") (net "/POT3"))
 (segment (start 118.825 59.325) (end 126.805 59.325) (width 0.25) (layer "F.Cu") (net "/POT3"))
 (segment (start 126.805 59.325) (end 133.98 66.5) (width 0.25) (layer "F.Cu") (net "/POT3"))
 (segment (start 91.275 71.105) (end 95.88 66.5) (width 1) (layer "F.Cu") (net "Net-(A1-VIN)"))
 (segment (start 91.275 90.225) (end 91.275 71.105) (width 1) (layer "F.Cu") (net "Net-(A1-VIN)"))
 (segment (start 89.5 92) (end 91.275 90.225) (width 1) (layer "F.Cu") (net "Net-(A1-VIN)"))
 (segment (start 107.405 81.253299) (end 120.983299 67.675) (width 0.25) (layer "B.Cu") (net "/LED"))
 (segment (start 127.725 67.675) (end 128.9 66.5) (width 0.25) (layer "B.Cu") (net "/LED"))
 (segment (start 103.88 87.5) (end 107.405 83.975) (width 0.25) (layer "B.Cu") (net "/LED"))
 (segment (start 120.983299 67.675) (end 127.725 67.675) (width 0.25) (layer "B.Cu") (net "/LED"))
 (segment (start 107.405 83.975) (end 107.405 81.253299) (width 0.25) (layer "B.Cu") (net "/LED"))
 (segment (start 127.725 87.425) (end 127.725 70.215) (width 0.25) (layer "F.Cu") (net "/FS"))
 (segment (start 127.8 87.5) (end 127.725 87.425) (width 0.25) (layer "F.Cu") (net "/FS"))
 (segment (start 127.725 70.215) (end 131.44 66.5) (width 0.25) (layer "F.Cu") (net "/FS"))
 (segment (start 137.5 65.52) (end 136.52 66.5) (width 0.25) (layer "F.Cu") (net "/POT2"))
 (segment (start 137.5 57.5) (end 137.5 65.52) (width 0.25) (layer "F.Cu") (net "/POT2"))
 (segment (start 99 98) (end 119.279899 98) (width 0.25) (layer "F.Cu") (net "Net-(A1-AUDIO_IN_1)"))
 (segment (start 131.44 85.839899) (end 131.44 81.74) (width 0.25) (layer "F.Cu") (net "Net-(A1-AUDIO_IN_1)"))
 (segment (start 119.279899 98) (end 131.44 85.839899) (width 0.25) (layer "F.Cu") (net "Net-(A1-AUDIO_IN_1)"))
 (segment (start 140 85.22) (end 136.52 81.74) (width 0.25) (layer "F.Cu") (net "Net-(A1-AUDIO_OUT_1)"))
 (segment (start 140 98) (end 140 85.22) (width 0.25) (layer "F.Cu") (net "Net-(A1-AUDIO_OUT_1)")))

